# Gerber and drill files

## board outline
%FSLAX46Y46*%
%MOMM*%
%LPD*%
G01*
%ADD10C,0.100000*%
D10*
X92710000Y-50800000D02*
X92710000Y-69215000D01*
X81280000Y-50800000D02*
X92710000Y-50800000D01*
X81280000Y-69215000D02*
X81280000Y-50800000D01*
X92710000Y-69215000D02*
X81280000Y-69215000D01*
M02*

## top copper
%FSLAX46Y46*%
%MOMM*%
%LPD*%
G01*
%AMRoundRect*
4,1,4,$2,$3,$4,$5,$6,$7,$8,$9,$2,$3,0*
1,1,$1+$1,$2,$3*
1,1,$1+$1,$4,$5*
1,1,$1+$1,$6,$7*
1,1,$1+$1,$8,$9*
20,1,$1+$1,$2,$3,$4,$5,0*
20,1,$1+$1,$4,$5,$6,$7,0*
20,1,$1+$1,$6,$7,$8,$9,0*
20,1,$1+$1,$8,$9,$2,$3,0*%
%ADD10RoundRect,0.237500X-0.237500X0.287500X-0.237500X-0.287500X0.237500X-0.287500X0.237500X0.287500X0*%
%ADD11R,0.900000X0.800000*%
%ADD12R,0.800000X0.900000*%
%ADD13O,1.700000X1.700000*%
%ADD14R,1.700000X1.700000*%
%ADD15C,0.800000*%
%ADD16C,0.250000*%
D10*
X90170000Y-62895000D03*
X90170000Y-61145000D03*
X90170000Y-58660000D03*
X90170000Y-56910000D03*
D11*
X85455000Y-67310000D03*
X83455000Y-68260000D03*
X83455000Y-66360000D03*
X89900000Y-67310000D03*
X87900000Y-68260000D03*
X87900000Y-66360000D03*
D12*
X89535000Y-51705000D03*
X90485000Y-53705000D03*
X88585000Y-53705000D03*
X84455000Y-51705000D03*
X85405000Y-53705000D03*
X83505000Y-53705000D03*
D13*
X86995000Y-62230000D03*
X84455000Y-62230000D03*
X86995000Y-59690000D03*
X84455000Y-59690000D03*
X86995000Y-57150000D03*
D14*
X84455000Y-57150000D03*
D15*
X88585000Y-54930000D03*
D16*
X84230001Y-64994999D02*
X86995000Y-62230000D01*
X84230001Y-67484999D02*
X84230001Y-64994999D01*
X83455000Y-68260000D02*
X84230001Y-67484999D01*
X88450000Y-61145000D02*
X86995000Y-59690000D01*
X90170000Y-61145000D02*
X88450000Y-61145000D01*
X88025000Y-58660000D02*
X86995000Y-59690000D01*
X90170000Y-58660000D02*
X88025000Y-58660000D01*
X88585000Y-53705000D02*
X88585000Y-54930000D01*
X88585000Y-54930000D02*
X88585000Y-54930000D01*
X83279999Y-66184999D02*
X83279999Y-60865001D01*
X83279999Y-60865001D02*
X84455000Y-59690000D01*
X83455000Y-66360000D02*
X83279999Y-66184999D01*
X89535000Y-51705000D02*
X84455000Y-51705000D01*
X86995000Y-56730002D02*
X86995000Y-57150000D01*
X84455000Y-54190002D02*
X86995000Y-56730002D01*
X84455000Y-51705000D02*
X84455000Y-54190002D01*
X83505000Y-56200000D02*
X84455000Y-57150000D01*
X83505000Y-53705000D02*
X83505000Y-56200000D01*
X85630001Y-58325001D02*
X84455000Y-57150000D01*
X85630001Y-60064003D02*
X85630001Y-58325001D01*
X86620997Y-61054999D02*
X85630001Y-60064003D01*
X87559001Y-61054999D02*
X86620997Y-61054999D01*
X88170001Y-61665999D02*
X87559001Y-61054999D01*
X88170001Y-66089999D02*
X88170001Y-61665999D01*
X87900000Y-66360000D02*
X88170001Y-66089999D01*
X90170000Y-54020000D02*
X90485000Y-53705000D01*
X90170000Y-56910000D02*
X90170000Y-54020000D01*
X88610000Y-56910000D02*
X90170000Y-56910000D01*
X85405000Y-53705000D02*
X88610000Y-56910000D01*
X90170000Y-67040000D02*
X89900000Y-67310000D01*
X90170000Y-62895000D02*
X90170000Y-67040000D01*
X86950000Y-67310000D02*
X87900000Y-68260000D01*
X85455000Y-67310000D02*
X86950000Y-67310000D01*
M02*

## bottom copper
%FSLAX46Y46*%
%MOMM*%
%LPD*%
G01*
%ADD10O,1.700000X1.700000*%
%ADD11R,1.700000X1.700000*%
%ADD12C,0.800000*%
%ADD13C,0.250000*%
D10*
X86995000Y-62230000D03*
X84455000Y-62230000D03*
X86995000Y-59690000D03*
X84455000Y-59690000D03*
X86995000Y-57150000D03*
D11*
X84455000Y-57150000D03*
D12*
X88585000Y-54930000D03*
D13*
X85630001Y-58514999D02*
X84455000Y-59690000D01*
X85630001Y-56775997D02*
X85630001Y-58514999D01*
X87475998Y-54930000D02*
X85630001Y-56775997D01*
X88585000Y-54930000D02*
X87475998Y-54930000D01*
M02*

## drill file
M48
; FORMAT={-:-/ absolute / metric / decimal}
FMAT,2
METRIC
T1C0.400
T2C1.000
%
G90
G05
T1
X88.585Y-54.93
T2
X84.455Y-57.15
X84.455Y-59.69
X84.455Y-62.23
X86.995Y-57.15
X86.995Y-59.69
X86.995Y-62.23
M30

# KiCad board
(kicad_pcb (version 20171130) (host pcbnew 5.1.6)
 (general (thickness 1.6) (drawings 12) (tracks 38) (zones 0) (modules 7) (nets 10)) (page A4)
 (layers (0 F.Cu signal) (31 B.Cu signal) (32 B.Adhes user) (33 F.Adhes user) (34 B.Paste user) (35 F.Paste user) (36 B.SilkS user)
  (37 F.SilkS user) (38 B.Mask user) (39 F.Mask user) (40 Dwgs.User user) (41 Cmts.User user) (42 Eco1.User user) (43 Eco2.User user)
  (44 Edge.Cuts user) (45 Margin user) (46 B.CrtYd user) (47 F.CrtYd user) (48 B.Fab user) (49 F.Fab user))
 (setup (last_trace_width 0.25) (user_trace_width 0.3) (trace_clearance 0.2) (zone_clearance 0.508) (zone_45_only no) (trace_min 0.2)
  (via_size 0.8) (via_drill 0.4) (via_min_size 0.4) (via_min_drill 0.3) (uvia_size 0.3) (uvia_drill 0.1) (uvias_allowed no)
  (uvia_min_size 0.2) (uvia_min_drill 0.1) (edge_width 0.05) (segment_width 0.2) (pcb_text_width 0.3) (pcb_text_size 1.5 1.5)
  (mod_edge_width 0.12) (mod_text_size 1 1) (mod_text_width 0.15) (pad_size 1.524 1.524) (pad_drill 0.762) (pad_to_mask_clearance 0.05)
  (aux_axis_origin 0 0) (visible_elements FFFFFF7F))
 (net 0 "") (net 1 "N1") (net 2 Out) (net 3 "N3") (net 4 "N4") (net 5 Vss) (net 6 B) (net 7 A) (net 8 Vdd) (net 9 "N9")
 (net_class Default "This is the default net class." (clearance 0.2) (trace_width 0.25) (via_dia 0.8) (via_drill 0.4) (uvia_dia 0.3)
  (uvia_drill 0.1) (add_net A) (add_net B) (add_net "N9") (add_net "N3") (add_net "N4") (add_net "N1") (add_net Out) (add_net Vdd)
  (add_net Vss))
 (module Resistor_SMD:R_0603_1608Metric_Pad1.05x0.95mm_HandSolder (layer F.Cu) (at 90.17 62.02 270)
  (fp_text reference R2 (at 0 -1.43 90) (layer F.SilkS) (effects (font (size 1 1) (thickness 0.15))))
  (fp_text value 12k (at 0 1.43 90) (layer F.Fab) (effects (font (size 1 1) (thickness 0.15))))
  (pad 2 smd roundrect (at 0.875 0 270) (size 1.05 0.95) (layers F.Cu F.Paste F.Mask) (roundrect_rratio 0.25) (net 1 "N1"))
  (pad 1 smd roundrect (at -0.875 0 270) (size 1.05 0.95) (layers F.Cu F.Paste F.Mask) (roundrect_rratio 0.25) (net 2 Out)))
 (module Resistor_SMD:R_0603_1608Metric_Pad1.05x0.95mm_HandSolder (layer F.Cu) (at 90.17 57.785 270)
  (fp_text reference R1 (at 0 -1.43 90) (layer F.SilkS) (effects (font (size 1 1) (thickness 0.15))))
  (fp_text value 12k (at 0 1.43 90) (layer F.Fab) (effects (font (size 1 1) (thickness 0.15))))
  (pad 2 smd roundrect (at 0.875 0 270) (size 1.05 0.95) (layers F.Cu F.Paste F.Mask) (roundrect_rratio 0.25) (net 2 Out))
  (pad 1 smd roundrect (at -0.875 0 270) (size 1.05 0.95) (layers F.Cu F.Paste F.Mask) (roundrect_rratio 0.25) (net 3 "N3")))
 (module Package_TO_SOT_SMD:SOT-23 (layer F.Cu) (at 84.455 67.31)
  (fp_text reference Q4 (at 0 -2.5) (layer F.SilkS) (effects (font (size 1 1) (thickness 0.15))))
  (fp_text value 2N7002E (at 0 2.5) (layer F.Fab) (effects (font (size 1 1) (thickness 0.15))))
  (pad 3 smd rect (at 1 0) (size 0.9 0.8) (layers F.Cu F.Paste F.Mask) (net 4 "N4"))
  (pad 2 smd rect (at -1 0.95) (size 0.9 0.8) (layers F.Cu F.Paste F.Mask) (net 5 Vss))
  (pad 1 smd rect (at -1 -0.95) (size 0.9 0.8) (layers F.Cu F.Paste F.Mask) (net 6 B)))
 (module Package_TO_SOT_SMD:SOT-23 (layer F.Cu) (at 88.9 67.31)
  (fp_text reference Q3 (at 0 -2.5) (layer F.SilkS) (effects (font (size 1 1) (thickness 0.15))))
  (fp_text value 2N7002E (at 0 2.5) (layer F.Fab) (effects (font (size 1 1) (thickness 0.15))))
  (pad 3 smd rect (at 1 0) (size 0.9 0.8) (layers F.Cu F.Paste F.Mask) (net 1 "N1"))
  (pad 2 smd rect (at -1 0.95) (size 0.9 0.8) (layers F.Cu F.Paste F.Mask) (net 4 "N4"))
  (pad 1 smd rect (at -1 -0.95) (size 0.9 0.8) (layers F.Cu F.Paste F.Mask) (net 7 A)))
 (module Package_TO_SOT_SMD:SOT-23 (layer F.Cu) (at 89.535 52.705 90)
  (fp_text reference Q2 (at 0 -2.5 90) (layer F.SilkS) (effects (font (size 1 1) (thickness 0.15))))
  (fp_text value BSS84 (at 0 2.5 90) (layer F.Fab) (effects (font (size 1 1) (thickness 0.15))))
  (pad 3 smd rect (at 1 0 90) (size 0.9 0.8) (layers F.Cu F.Paste F.Mask) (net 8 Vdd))
  (pad 2 smd rect (at -1 0.95 90) (size 0.9 0.8) (layers F.Cu F.Paste F.Mask) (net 3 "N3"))
  (pad 1 smd rect (at -1 -0.95 90) (size 0.9 0.8) (layers F.Cu F.Paste F.Mask) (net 6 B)))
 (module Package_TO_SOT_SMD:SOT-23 (layer F.Cu) (at 84.455 52.705 90)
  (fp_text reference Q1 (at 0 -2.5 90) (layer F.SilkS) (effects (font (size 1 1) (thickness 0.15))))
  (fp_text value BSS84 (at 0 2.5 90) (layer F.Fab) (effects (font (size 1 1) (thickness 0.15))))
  (pad 3 smd rect (at 1 0 90) (size 0.9 0.8) (layers F.Cu F.Paste F.Mask) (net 8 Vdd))
  (pad 2 smd rect (at -1 0.95 90) (size 0.9 0.8) (layers F.Cu F.Paste F.Mask) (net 3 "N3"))
  (pad 1 smd rect (at -1 -0.95 90) (size 0.9 0.8) (layers F.Cu F.Paste F.Mask) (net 7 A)))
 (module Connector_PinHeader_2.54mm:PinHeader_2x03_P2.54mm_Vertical (layer F.Cu) (at 84.455 57.15)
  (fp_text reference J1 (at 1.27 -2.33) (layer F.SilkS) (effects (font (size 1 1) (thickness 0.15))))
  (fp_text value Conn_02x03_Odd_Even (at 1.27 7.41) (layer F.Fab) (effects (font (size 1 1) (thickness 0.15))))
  (pad 6 thru_hole oval (at 2.54 5.08) (size 1.7 1.7) (drill 1) (layers *.Cu *.Mask) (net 5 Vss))
  (pad 5 thru_hole oval (at 0 5.08) (size 1.7 1.7) (drill 1) (layers *.Cu *.Mask) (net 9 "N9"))
  (pad 4 thru_hole oval (at 2.54 2.54) (size 1.7 1.7) (drill 1) (layers *.Cu *.Mask) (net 2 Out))
  (pad 3 thru_hole oval (at 0 2.54) (size 1.7 1.7) (drill 1) (layers *.Cu *.Mask) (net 6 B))
  (pad 2 thru_hole oval (at 2.54 0) (size 1.7 1.7) (drill 1) (layers *.Cu *.Mask) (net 8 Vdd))
  (pad 1 thru_hole rect (at 0 0) (size 1.7 1.7) (drill 1) (layers *.Cu *.Mask) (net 7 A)))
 (gr_line (start 92.71 50.8) (end 92.71 69.215) (layer Edge.Cuts) (width 0.1))
 (gr_line (start 81.28 50.8) (end 92.71 50.8) (layer Edge.Cuts) (width 0.1))
 (gr_line (start 81.28 69.215) (end 81.28 50.8) (layer Edge.Cuts) (width 0.1))
 (gr_line (start 92.71 69.215) (end 81.28 69.215) (layer Edge.Cuts) (width 0.1))
 (segment (start 84.230001 64.994999) (end 86.995 62.23) (width 0.25) (layer F.Cu) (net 5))
 (segment (start 84.230001 67.484999) (end 84.230001 64.994999) (width 0.25) (layer F.Cu) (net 5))
 (segment (start 83.455 68.26) (end 84.230001 67.484999) (width 0.25) (layer F.Cu) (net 5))
 (segment (start 88.45 61.145) (end 86.995 59.69) (width 0.25) (layer F.Cu) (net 2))
 (segment (start 90.17 61.145) (end 88.45 61.145) (width 0.25) (layer F.Cu) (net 2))
 (segment (start 88.025 58.66) (end 86.995 59.69) (width 0.25) (layer F.Cu) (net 2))
 (segment (start 90.17 58.66) (end 88.025 58.66) (width 0.25) (layer F.Cu) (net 2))
 (segment (start 88.585 53.705) (end 88.585 54.93) (width 0.25) (layer F.Cu) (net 6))
 (segment (start 88.585 54.93) (end 88.585 54.93) (width 0.25) (layer F.Cu) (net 6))
 (via (at 88.585 54.93) (size 0.8) (drill 0.4) (layers F.Cu B.Cu) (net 6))
 (segment (start 85.630001 58.514999) (end 84.455 59.69) (width 0.25) (layer B.Cu) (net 6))
 (segment (start 85.630001 56.775997) (end 85.630001 58.514999) (width 0.25) (layer B.Cu) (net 6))
 (segment (start 87.475998 54.93) (end 85.630001 56.775997) (width 0.25) (layer B.Cu) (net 6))
 (segment (start 88.585 54.93) (end 87.475998 54.93) (width 0.25) (layer B.Cu) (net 6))
 (segment (start 83.279999 66.184999) (end 83.279999 60.865001) (width 0.25) (layer F.Cu) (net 6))
 (segment (start 83.279999 60.865001) (end 84.455 59.69) (width 0.25) (layer F.Cu) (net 6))
 (segment (start 83.455 66.36) (end 83.279999 66.184999) (width 0.25) (layer F.Cu) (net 6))
 (segment (start 89.535 51.705) (end 84.455 51.705) (width 0.25) (layer F.Cu) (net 8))
 (segment (start 86.995 56.730002) (end 86.995 57.15) (width 0.25) (layer F.Cu) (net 8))
 (segment (start 84.455 54.190002) (end 86.995 56.730002) (width 0.25) (layer F.Cu) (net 8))
 (segment (start 84.455 51.705) (end 84.455 54.190002) (width 0.25) (layer F.Cu) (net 8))
 (segment (start 83.505 56.2) (end 84.455 57.15) (width 0.25) (layer F.Cu) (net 7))
 (segment (start 83.505 53.705) (end 83.505 56.2) (width 0.25) (layer F.Cu) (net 7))
 (segment (start 85.630001 58.325001) (end 84.455 57.15) (width 0.25) (layer F.Cu) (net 7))
 (segment (start 85.630001 60.064003) (end 85.630001 58.325001) (width 0.25) (layer F.Cu) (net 7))
 (segment (start 86.620997 61.054999) (end 85.630001 60.064003) (width 0.25) (layer F.Cu) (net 7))
 (segment (start 87.559001 61.054999) (end 86.620997 61.054999) (width 0.25) (layer F.Cu) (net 7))
 (segment (start 88.170001 61.665999) (end 87.559001 61.054999) (width 0.25) (layer F.Cu) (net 7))
 (segment (start 88.170001 66.089999) (end 88.170001 61.665999) (width 0.25) (layer F.Cu) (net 7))
 (segment (start 87.9 66.36) (end 88.170001 66.089999) (width 0.25) (layer F.Cu) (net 7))
 (segment (start 90.17 54.02) (end 90.485 53.705) (width 0.25) (layer F.Cu) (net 3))
 (segment (start 90.17 56.91) (end 90.17 54.02) (width 0.25) (layer F.Cu) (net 3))
 (segment (start 88.61 56.91) (end 90.17 56.91) (width 0.25) (layer F.Cu) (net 3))
 (segment (start 85.405 53.705) (end 88.61 56.91) (width 0.25) (layer F.Cu) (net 3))
 (segment (start 90.17 67.04) (end 89.9 67.31) (width 0.25) (layer F.Cu) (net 1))
 (segment (start 90.17 62.895) (end 90.17 67.04) (width 0.25) (layer F.Cu) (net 1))
 (segment (start 86.95 67.31) (end 87.9 68.26) (width 0.25) (layer F.Cu) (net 4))
 (segment (start 85.455 67.31) (end 86.95 67.31) (width 0.25) (layer F.Cu) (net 4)))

